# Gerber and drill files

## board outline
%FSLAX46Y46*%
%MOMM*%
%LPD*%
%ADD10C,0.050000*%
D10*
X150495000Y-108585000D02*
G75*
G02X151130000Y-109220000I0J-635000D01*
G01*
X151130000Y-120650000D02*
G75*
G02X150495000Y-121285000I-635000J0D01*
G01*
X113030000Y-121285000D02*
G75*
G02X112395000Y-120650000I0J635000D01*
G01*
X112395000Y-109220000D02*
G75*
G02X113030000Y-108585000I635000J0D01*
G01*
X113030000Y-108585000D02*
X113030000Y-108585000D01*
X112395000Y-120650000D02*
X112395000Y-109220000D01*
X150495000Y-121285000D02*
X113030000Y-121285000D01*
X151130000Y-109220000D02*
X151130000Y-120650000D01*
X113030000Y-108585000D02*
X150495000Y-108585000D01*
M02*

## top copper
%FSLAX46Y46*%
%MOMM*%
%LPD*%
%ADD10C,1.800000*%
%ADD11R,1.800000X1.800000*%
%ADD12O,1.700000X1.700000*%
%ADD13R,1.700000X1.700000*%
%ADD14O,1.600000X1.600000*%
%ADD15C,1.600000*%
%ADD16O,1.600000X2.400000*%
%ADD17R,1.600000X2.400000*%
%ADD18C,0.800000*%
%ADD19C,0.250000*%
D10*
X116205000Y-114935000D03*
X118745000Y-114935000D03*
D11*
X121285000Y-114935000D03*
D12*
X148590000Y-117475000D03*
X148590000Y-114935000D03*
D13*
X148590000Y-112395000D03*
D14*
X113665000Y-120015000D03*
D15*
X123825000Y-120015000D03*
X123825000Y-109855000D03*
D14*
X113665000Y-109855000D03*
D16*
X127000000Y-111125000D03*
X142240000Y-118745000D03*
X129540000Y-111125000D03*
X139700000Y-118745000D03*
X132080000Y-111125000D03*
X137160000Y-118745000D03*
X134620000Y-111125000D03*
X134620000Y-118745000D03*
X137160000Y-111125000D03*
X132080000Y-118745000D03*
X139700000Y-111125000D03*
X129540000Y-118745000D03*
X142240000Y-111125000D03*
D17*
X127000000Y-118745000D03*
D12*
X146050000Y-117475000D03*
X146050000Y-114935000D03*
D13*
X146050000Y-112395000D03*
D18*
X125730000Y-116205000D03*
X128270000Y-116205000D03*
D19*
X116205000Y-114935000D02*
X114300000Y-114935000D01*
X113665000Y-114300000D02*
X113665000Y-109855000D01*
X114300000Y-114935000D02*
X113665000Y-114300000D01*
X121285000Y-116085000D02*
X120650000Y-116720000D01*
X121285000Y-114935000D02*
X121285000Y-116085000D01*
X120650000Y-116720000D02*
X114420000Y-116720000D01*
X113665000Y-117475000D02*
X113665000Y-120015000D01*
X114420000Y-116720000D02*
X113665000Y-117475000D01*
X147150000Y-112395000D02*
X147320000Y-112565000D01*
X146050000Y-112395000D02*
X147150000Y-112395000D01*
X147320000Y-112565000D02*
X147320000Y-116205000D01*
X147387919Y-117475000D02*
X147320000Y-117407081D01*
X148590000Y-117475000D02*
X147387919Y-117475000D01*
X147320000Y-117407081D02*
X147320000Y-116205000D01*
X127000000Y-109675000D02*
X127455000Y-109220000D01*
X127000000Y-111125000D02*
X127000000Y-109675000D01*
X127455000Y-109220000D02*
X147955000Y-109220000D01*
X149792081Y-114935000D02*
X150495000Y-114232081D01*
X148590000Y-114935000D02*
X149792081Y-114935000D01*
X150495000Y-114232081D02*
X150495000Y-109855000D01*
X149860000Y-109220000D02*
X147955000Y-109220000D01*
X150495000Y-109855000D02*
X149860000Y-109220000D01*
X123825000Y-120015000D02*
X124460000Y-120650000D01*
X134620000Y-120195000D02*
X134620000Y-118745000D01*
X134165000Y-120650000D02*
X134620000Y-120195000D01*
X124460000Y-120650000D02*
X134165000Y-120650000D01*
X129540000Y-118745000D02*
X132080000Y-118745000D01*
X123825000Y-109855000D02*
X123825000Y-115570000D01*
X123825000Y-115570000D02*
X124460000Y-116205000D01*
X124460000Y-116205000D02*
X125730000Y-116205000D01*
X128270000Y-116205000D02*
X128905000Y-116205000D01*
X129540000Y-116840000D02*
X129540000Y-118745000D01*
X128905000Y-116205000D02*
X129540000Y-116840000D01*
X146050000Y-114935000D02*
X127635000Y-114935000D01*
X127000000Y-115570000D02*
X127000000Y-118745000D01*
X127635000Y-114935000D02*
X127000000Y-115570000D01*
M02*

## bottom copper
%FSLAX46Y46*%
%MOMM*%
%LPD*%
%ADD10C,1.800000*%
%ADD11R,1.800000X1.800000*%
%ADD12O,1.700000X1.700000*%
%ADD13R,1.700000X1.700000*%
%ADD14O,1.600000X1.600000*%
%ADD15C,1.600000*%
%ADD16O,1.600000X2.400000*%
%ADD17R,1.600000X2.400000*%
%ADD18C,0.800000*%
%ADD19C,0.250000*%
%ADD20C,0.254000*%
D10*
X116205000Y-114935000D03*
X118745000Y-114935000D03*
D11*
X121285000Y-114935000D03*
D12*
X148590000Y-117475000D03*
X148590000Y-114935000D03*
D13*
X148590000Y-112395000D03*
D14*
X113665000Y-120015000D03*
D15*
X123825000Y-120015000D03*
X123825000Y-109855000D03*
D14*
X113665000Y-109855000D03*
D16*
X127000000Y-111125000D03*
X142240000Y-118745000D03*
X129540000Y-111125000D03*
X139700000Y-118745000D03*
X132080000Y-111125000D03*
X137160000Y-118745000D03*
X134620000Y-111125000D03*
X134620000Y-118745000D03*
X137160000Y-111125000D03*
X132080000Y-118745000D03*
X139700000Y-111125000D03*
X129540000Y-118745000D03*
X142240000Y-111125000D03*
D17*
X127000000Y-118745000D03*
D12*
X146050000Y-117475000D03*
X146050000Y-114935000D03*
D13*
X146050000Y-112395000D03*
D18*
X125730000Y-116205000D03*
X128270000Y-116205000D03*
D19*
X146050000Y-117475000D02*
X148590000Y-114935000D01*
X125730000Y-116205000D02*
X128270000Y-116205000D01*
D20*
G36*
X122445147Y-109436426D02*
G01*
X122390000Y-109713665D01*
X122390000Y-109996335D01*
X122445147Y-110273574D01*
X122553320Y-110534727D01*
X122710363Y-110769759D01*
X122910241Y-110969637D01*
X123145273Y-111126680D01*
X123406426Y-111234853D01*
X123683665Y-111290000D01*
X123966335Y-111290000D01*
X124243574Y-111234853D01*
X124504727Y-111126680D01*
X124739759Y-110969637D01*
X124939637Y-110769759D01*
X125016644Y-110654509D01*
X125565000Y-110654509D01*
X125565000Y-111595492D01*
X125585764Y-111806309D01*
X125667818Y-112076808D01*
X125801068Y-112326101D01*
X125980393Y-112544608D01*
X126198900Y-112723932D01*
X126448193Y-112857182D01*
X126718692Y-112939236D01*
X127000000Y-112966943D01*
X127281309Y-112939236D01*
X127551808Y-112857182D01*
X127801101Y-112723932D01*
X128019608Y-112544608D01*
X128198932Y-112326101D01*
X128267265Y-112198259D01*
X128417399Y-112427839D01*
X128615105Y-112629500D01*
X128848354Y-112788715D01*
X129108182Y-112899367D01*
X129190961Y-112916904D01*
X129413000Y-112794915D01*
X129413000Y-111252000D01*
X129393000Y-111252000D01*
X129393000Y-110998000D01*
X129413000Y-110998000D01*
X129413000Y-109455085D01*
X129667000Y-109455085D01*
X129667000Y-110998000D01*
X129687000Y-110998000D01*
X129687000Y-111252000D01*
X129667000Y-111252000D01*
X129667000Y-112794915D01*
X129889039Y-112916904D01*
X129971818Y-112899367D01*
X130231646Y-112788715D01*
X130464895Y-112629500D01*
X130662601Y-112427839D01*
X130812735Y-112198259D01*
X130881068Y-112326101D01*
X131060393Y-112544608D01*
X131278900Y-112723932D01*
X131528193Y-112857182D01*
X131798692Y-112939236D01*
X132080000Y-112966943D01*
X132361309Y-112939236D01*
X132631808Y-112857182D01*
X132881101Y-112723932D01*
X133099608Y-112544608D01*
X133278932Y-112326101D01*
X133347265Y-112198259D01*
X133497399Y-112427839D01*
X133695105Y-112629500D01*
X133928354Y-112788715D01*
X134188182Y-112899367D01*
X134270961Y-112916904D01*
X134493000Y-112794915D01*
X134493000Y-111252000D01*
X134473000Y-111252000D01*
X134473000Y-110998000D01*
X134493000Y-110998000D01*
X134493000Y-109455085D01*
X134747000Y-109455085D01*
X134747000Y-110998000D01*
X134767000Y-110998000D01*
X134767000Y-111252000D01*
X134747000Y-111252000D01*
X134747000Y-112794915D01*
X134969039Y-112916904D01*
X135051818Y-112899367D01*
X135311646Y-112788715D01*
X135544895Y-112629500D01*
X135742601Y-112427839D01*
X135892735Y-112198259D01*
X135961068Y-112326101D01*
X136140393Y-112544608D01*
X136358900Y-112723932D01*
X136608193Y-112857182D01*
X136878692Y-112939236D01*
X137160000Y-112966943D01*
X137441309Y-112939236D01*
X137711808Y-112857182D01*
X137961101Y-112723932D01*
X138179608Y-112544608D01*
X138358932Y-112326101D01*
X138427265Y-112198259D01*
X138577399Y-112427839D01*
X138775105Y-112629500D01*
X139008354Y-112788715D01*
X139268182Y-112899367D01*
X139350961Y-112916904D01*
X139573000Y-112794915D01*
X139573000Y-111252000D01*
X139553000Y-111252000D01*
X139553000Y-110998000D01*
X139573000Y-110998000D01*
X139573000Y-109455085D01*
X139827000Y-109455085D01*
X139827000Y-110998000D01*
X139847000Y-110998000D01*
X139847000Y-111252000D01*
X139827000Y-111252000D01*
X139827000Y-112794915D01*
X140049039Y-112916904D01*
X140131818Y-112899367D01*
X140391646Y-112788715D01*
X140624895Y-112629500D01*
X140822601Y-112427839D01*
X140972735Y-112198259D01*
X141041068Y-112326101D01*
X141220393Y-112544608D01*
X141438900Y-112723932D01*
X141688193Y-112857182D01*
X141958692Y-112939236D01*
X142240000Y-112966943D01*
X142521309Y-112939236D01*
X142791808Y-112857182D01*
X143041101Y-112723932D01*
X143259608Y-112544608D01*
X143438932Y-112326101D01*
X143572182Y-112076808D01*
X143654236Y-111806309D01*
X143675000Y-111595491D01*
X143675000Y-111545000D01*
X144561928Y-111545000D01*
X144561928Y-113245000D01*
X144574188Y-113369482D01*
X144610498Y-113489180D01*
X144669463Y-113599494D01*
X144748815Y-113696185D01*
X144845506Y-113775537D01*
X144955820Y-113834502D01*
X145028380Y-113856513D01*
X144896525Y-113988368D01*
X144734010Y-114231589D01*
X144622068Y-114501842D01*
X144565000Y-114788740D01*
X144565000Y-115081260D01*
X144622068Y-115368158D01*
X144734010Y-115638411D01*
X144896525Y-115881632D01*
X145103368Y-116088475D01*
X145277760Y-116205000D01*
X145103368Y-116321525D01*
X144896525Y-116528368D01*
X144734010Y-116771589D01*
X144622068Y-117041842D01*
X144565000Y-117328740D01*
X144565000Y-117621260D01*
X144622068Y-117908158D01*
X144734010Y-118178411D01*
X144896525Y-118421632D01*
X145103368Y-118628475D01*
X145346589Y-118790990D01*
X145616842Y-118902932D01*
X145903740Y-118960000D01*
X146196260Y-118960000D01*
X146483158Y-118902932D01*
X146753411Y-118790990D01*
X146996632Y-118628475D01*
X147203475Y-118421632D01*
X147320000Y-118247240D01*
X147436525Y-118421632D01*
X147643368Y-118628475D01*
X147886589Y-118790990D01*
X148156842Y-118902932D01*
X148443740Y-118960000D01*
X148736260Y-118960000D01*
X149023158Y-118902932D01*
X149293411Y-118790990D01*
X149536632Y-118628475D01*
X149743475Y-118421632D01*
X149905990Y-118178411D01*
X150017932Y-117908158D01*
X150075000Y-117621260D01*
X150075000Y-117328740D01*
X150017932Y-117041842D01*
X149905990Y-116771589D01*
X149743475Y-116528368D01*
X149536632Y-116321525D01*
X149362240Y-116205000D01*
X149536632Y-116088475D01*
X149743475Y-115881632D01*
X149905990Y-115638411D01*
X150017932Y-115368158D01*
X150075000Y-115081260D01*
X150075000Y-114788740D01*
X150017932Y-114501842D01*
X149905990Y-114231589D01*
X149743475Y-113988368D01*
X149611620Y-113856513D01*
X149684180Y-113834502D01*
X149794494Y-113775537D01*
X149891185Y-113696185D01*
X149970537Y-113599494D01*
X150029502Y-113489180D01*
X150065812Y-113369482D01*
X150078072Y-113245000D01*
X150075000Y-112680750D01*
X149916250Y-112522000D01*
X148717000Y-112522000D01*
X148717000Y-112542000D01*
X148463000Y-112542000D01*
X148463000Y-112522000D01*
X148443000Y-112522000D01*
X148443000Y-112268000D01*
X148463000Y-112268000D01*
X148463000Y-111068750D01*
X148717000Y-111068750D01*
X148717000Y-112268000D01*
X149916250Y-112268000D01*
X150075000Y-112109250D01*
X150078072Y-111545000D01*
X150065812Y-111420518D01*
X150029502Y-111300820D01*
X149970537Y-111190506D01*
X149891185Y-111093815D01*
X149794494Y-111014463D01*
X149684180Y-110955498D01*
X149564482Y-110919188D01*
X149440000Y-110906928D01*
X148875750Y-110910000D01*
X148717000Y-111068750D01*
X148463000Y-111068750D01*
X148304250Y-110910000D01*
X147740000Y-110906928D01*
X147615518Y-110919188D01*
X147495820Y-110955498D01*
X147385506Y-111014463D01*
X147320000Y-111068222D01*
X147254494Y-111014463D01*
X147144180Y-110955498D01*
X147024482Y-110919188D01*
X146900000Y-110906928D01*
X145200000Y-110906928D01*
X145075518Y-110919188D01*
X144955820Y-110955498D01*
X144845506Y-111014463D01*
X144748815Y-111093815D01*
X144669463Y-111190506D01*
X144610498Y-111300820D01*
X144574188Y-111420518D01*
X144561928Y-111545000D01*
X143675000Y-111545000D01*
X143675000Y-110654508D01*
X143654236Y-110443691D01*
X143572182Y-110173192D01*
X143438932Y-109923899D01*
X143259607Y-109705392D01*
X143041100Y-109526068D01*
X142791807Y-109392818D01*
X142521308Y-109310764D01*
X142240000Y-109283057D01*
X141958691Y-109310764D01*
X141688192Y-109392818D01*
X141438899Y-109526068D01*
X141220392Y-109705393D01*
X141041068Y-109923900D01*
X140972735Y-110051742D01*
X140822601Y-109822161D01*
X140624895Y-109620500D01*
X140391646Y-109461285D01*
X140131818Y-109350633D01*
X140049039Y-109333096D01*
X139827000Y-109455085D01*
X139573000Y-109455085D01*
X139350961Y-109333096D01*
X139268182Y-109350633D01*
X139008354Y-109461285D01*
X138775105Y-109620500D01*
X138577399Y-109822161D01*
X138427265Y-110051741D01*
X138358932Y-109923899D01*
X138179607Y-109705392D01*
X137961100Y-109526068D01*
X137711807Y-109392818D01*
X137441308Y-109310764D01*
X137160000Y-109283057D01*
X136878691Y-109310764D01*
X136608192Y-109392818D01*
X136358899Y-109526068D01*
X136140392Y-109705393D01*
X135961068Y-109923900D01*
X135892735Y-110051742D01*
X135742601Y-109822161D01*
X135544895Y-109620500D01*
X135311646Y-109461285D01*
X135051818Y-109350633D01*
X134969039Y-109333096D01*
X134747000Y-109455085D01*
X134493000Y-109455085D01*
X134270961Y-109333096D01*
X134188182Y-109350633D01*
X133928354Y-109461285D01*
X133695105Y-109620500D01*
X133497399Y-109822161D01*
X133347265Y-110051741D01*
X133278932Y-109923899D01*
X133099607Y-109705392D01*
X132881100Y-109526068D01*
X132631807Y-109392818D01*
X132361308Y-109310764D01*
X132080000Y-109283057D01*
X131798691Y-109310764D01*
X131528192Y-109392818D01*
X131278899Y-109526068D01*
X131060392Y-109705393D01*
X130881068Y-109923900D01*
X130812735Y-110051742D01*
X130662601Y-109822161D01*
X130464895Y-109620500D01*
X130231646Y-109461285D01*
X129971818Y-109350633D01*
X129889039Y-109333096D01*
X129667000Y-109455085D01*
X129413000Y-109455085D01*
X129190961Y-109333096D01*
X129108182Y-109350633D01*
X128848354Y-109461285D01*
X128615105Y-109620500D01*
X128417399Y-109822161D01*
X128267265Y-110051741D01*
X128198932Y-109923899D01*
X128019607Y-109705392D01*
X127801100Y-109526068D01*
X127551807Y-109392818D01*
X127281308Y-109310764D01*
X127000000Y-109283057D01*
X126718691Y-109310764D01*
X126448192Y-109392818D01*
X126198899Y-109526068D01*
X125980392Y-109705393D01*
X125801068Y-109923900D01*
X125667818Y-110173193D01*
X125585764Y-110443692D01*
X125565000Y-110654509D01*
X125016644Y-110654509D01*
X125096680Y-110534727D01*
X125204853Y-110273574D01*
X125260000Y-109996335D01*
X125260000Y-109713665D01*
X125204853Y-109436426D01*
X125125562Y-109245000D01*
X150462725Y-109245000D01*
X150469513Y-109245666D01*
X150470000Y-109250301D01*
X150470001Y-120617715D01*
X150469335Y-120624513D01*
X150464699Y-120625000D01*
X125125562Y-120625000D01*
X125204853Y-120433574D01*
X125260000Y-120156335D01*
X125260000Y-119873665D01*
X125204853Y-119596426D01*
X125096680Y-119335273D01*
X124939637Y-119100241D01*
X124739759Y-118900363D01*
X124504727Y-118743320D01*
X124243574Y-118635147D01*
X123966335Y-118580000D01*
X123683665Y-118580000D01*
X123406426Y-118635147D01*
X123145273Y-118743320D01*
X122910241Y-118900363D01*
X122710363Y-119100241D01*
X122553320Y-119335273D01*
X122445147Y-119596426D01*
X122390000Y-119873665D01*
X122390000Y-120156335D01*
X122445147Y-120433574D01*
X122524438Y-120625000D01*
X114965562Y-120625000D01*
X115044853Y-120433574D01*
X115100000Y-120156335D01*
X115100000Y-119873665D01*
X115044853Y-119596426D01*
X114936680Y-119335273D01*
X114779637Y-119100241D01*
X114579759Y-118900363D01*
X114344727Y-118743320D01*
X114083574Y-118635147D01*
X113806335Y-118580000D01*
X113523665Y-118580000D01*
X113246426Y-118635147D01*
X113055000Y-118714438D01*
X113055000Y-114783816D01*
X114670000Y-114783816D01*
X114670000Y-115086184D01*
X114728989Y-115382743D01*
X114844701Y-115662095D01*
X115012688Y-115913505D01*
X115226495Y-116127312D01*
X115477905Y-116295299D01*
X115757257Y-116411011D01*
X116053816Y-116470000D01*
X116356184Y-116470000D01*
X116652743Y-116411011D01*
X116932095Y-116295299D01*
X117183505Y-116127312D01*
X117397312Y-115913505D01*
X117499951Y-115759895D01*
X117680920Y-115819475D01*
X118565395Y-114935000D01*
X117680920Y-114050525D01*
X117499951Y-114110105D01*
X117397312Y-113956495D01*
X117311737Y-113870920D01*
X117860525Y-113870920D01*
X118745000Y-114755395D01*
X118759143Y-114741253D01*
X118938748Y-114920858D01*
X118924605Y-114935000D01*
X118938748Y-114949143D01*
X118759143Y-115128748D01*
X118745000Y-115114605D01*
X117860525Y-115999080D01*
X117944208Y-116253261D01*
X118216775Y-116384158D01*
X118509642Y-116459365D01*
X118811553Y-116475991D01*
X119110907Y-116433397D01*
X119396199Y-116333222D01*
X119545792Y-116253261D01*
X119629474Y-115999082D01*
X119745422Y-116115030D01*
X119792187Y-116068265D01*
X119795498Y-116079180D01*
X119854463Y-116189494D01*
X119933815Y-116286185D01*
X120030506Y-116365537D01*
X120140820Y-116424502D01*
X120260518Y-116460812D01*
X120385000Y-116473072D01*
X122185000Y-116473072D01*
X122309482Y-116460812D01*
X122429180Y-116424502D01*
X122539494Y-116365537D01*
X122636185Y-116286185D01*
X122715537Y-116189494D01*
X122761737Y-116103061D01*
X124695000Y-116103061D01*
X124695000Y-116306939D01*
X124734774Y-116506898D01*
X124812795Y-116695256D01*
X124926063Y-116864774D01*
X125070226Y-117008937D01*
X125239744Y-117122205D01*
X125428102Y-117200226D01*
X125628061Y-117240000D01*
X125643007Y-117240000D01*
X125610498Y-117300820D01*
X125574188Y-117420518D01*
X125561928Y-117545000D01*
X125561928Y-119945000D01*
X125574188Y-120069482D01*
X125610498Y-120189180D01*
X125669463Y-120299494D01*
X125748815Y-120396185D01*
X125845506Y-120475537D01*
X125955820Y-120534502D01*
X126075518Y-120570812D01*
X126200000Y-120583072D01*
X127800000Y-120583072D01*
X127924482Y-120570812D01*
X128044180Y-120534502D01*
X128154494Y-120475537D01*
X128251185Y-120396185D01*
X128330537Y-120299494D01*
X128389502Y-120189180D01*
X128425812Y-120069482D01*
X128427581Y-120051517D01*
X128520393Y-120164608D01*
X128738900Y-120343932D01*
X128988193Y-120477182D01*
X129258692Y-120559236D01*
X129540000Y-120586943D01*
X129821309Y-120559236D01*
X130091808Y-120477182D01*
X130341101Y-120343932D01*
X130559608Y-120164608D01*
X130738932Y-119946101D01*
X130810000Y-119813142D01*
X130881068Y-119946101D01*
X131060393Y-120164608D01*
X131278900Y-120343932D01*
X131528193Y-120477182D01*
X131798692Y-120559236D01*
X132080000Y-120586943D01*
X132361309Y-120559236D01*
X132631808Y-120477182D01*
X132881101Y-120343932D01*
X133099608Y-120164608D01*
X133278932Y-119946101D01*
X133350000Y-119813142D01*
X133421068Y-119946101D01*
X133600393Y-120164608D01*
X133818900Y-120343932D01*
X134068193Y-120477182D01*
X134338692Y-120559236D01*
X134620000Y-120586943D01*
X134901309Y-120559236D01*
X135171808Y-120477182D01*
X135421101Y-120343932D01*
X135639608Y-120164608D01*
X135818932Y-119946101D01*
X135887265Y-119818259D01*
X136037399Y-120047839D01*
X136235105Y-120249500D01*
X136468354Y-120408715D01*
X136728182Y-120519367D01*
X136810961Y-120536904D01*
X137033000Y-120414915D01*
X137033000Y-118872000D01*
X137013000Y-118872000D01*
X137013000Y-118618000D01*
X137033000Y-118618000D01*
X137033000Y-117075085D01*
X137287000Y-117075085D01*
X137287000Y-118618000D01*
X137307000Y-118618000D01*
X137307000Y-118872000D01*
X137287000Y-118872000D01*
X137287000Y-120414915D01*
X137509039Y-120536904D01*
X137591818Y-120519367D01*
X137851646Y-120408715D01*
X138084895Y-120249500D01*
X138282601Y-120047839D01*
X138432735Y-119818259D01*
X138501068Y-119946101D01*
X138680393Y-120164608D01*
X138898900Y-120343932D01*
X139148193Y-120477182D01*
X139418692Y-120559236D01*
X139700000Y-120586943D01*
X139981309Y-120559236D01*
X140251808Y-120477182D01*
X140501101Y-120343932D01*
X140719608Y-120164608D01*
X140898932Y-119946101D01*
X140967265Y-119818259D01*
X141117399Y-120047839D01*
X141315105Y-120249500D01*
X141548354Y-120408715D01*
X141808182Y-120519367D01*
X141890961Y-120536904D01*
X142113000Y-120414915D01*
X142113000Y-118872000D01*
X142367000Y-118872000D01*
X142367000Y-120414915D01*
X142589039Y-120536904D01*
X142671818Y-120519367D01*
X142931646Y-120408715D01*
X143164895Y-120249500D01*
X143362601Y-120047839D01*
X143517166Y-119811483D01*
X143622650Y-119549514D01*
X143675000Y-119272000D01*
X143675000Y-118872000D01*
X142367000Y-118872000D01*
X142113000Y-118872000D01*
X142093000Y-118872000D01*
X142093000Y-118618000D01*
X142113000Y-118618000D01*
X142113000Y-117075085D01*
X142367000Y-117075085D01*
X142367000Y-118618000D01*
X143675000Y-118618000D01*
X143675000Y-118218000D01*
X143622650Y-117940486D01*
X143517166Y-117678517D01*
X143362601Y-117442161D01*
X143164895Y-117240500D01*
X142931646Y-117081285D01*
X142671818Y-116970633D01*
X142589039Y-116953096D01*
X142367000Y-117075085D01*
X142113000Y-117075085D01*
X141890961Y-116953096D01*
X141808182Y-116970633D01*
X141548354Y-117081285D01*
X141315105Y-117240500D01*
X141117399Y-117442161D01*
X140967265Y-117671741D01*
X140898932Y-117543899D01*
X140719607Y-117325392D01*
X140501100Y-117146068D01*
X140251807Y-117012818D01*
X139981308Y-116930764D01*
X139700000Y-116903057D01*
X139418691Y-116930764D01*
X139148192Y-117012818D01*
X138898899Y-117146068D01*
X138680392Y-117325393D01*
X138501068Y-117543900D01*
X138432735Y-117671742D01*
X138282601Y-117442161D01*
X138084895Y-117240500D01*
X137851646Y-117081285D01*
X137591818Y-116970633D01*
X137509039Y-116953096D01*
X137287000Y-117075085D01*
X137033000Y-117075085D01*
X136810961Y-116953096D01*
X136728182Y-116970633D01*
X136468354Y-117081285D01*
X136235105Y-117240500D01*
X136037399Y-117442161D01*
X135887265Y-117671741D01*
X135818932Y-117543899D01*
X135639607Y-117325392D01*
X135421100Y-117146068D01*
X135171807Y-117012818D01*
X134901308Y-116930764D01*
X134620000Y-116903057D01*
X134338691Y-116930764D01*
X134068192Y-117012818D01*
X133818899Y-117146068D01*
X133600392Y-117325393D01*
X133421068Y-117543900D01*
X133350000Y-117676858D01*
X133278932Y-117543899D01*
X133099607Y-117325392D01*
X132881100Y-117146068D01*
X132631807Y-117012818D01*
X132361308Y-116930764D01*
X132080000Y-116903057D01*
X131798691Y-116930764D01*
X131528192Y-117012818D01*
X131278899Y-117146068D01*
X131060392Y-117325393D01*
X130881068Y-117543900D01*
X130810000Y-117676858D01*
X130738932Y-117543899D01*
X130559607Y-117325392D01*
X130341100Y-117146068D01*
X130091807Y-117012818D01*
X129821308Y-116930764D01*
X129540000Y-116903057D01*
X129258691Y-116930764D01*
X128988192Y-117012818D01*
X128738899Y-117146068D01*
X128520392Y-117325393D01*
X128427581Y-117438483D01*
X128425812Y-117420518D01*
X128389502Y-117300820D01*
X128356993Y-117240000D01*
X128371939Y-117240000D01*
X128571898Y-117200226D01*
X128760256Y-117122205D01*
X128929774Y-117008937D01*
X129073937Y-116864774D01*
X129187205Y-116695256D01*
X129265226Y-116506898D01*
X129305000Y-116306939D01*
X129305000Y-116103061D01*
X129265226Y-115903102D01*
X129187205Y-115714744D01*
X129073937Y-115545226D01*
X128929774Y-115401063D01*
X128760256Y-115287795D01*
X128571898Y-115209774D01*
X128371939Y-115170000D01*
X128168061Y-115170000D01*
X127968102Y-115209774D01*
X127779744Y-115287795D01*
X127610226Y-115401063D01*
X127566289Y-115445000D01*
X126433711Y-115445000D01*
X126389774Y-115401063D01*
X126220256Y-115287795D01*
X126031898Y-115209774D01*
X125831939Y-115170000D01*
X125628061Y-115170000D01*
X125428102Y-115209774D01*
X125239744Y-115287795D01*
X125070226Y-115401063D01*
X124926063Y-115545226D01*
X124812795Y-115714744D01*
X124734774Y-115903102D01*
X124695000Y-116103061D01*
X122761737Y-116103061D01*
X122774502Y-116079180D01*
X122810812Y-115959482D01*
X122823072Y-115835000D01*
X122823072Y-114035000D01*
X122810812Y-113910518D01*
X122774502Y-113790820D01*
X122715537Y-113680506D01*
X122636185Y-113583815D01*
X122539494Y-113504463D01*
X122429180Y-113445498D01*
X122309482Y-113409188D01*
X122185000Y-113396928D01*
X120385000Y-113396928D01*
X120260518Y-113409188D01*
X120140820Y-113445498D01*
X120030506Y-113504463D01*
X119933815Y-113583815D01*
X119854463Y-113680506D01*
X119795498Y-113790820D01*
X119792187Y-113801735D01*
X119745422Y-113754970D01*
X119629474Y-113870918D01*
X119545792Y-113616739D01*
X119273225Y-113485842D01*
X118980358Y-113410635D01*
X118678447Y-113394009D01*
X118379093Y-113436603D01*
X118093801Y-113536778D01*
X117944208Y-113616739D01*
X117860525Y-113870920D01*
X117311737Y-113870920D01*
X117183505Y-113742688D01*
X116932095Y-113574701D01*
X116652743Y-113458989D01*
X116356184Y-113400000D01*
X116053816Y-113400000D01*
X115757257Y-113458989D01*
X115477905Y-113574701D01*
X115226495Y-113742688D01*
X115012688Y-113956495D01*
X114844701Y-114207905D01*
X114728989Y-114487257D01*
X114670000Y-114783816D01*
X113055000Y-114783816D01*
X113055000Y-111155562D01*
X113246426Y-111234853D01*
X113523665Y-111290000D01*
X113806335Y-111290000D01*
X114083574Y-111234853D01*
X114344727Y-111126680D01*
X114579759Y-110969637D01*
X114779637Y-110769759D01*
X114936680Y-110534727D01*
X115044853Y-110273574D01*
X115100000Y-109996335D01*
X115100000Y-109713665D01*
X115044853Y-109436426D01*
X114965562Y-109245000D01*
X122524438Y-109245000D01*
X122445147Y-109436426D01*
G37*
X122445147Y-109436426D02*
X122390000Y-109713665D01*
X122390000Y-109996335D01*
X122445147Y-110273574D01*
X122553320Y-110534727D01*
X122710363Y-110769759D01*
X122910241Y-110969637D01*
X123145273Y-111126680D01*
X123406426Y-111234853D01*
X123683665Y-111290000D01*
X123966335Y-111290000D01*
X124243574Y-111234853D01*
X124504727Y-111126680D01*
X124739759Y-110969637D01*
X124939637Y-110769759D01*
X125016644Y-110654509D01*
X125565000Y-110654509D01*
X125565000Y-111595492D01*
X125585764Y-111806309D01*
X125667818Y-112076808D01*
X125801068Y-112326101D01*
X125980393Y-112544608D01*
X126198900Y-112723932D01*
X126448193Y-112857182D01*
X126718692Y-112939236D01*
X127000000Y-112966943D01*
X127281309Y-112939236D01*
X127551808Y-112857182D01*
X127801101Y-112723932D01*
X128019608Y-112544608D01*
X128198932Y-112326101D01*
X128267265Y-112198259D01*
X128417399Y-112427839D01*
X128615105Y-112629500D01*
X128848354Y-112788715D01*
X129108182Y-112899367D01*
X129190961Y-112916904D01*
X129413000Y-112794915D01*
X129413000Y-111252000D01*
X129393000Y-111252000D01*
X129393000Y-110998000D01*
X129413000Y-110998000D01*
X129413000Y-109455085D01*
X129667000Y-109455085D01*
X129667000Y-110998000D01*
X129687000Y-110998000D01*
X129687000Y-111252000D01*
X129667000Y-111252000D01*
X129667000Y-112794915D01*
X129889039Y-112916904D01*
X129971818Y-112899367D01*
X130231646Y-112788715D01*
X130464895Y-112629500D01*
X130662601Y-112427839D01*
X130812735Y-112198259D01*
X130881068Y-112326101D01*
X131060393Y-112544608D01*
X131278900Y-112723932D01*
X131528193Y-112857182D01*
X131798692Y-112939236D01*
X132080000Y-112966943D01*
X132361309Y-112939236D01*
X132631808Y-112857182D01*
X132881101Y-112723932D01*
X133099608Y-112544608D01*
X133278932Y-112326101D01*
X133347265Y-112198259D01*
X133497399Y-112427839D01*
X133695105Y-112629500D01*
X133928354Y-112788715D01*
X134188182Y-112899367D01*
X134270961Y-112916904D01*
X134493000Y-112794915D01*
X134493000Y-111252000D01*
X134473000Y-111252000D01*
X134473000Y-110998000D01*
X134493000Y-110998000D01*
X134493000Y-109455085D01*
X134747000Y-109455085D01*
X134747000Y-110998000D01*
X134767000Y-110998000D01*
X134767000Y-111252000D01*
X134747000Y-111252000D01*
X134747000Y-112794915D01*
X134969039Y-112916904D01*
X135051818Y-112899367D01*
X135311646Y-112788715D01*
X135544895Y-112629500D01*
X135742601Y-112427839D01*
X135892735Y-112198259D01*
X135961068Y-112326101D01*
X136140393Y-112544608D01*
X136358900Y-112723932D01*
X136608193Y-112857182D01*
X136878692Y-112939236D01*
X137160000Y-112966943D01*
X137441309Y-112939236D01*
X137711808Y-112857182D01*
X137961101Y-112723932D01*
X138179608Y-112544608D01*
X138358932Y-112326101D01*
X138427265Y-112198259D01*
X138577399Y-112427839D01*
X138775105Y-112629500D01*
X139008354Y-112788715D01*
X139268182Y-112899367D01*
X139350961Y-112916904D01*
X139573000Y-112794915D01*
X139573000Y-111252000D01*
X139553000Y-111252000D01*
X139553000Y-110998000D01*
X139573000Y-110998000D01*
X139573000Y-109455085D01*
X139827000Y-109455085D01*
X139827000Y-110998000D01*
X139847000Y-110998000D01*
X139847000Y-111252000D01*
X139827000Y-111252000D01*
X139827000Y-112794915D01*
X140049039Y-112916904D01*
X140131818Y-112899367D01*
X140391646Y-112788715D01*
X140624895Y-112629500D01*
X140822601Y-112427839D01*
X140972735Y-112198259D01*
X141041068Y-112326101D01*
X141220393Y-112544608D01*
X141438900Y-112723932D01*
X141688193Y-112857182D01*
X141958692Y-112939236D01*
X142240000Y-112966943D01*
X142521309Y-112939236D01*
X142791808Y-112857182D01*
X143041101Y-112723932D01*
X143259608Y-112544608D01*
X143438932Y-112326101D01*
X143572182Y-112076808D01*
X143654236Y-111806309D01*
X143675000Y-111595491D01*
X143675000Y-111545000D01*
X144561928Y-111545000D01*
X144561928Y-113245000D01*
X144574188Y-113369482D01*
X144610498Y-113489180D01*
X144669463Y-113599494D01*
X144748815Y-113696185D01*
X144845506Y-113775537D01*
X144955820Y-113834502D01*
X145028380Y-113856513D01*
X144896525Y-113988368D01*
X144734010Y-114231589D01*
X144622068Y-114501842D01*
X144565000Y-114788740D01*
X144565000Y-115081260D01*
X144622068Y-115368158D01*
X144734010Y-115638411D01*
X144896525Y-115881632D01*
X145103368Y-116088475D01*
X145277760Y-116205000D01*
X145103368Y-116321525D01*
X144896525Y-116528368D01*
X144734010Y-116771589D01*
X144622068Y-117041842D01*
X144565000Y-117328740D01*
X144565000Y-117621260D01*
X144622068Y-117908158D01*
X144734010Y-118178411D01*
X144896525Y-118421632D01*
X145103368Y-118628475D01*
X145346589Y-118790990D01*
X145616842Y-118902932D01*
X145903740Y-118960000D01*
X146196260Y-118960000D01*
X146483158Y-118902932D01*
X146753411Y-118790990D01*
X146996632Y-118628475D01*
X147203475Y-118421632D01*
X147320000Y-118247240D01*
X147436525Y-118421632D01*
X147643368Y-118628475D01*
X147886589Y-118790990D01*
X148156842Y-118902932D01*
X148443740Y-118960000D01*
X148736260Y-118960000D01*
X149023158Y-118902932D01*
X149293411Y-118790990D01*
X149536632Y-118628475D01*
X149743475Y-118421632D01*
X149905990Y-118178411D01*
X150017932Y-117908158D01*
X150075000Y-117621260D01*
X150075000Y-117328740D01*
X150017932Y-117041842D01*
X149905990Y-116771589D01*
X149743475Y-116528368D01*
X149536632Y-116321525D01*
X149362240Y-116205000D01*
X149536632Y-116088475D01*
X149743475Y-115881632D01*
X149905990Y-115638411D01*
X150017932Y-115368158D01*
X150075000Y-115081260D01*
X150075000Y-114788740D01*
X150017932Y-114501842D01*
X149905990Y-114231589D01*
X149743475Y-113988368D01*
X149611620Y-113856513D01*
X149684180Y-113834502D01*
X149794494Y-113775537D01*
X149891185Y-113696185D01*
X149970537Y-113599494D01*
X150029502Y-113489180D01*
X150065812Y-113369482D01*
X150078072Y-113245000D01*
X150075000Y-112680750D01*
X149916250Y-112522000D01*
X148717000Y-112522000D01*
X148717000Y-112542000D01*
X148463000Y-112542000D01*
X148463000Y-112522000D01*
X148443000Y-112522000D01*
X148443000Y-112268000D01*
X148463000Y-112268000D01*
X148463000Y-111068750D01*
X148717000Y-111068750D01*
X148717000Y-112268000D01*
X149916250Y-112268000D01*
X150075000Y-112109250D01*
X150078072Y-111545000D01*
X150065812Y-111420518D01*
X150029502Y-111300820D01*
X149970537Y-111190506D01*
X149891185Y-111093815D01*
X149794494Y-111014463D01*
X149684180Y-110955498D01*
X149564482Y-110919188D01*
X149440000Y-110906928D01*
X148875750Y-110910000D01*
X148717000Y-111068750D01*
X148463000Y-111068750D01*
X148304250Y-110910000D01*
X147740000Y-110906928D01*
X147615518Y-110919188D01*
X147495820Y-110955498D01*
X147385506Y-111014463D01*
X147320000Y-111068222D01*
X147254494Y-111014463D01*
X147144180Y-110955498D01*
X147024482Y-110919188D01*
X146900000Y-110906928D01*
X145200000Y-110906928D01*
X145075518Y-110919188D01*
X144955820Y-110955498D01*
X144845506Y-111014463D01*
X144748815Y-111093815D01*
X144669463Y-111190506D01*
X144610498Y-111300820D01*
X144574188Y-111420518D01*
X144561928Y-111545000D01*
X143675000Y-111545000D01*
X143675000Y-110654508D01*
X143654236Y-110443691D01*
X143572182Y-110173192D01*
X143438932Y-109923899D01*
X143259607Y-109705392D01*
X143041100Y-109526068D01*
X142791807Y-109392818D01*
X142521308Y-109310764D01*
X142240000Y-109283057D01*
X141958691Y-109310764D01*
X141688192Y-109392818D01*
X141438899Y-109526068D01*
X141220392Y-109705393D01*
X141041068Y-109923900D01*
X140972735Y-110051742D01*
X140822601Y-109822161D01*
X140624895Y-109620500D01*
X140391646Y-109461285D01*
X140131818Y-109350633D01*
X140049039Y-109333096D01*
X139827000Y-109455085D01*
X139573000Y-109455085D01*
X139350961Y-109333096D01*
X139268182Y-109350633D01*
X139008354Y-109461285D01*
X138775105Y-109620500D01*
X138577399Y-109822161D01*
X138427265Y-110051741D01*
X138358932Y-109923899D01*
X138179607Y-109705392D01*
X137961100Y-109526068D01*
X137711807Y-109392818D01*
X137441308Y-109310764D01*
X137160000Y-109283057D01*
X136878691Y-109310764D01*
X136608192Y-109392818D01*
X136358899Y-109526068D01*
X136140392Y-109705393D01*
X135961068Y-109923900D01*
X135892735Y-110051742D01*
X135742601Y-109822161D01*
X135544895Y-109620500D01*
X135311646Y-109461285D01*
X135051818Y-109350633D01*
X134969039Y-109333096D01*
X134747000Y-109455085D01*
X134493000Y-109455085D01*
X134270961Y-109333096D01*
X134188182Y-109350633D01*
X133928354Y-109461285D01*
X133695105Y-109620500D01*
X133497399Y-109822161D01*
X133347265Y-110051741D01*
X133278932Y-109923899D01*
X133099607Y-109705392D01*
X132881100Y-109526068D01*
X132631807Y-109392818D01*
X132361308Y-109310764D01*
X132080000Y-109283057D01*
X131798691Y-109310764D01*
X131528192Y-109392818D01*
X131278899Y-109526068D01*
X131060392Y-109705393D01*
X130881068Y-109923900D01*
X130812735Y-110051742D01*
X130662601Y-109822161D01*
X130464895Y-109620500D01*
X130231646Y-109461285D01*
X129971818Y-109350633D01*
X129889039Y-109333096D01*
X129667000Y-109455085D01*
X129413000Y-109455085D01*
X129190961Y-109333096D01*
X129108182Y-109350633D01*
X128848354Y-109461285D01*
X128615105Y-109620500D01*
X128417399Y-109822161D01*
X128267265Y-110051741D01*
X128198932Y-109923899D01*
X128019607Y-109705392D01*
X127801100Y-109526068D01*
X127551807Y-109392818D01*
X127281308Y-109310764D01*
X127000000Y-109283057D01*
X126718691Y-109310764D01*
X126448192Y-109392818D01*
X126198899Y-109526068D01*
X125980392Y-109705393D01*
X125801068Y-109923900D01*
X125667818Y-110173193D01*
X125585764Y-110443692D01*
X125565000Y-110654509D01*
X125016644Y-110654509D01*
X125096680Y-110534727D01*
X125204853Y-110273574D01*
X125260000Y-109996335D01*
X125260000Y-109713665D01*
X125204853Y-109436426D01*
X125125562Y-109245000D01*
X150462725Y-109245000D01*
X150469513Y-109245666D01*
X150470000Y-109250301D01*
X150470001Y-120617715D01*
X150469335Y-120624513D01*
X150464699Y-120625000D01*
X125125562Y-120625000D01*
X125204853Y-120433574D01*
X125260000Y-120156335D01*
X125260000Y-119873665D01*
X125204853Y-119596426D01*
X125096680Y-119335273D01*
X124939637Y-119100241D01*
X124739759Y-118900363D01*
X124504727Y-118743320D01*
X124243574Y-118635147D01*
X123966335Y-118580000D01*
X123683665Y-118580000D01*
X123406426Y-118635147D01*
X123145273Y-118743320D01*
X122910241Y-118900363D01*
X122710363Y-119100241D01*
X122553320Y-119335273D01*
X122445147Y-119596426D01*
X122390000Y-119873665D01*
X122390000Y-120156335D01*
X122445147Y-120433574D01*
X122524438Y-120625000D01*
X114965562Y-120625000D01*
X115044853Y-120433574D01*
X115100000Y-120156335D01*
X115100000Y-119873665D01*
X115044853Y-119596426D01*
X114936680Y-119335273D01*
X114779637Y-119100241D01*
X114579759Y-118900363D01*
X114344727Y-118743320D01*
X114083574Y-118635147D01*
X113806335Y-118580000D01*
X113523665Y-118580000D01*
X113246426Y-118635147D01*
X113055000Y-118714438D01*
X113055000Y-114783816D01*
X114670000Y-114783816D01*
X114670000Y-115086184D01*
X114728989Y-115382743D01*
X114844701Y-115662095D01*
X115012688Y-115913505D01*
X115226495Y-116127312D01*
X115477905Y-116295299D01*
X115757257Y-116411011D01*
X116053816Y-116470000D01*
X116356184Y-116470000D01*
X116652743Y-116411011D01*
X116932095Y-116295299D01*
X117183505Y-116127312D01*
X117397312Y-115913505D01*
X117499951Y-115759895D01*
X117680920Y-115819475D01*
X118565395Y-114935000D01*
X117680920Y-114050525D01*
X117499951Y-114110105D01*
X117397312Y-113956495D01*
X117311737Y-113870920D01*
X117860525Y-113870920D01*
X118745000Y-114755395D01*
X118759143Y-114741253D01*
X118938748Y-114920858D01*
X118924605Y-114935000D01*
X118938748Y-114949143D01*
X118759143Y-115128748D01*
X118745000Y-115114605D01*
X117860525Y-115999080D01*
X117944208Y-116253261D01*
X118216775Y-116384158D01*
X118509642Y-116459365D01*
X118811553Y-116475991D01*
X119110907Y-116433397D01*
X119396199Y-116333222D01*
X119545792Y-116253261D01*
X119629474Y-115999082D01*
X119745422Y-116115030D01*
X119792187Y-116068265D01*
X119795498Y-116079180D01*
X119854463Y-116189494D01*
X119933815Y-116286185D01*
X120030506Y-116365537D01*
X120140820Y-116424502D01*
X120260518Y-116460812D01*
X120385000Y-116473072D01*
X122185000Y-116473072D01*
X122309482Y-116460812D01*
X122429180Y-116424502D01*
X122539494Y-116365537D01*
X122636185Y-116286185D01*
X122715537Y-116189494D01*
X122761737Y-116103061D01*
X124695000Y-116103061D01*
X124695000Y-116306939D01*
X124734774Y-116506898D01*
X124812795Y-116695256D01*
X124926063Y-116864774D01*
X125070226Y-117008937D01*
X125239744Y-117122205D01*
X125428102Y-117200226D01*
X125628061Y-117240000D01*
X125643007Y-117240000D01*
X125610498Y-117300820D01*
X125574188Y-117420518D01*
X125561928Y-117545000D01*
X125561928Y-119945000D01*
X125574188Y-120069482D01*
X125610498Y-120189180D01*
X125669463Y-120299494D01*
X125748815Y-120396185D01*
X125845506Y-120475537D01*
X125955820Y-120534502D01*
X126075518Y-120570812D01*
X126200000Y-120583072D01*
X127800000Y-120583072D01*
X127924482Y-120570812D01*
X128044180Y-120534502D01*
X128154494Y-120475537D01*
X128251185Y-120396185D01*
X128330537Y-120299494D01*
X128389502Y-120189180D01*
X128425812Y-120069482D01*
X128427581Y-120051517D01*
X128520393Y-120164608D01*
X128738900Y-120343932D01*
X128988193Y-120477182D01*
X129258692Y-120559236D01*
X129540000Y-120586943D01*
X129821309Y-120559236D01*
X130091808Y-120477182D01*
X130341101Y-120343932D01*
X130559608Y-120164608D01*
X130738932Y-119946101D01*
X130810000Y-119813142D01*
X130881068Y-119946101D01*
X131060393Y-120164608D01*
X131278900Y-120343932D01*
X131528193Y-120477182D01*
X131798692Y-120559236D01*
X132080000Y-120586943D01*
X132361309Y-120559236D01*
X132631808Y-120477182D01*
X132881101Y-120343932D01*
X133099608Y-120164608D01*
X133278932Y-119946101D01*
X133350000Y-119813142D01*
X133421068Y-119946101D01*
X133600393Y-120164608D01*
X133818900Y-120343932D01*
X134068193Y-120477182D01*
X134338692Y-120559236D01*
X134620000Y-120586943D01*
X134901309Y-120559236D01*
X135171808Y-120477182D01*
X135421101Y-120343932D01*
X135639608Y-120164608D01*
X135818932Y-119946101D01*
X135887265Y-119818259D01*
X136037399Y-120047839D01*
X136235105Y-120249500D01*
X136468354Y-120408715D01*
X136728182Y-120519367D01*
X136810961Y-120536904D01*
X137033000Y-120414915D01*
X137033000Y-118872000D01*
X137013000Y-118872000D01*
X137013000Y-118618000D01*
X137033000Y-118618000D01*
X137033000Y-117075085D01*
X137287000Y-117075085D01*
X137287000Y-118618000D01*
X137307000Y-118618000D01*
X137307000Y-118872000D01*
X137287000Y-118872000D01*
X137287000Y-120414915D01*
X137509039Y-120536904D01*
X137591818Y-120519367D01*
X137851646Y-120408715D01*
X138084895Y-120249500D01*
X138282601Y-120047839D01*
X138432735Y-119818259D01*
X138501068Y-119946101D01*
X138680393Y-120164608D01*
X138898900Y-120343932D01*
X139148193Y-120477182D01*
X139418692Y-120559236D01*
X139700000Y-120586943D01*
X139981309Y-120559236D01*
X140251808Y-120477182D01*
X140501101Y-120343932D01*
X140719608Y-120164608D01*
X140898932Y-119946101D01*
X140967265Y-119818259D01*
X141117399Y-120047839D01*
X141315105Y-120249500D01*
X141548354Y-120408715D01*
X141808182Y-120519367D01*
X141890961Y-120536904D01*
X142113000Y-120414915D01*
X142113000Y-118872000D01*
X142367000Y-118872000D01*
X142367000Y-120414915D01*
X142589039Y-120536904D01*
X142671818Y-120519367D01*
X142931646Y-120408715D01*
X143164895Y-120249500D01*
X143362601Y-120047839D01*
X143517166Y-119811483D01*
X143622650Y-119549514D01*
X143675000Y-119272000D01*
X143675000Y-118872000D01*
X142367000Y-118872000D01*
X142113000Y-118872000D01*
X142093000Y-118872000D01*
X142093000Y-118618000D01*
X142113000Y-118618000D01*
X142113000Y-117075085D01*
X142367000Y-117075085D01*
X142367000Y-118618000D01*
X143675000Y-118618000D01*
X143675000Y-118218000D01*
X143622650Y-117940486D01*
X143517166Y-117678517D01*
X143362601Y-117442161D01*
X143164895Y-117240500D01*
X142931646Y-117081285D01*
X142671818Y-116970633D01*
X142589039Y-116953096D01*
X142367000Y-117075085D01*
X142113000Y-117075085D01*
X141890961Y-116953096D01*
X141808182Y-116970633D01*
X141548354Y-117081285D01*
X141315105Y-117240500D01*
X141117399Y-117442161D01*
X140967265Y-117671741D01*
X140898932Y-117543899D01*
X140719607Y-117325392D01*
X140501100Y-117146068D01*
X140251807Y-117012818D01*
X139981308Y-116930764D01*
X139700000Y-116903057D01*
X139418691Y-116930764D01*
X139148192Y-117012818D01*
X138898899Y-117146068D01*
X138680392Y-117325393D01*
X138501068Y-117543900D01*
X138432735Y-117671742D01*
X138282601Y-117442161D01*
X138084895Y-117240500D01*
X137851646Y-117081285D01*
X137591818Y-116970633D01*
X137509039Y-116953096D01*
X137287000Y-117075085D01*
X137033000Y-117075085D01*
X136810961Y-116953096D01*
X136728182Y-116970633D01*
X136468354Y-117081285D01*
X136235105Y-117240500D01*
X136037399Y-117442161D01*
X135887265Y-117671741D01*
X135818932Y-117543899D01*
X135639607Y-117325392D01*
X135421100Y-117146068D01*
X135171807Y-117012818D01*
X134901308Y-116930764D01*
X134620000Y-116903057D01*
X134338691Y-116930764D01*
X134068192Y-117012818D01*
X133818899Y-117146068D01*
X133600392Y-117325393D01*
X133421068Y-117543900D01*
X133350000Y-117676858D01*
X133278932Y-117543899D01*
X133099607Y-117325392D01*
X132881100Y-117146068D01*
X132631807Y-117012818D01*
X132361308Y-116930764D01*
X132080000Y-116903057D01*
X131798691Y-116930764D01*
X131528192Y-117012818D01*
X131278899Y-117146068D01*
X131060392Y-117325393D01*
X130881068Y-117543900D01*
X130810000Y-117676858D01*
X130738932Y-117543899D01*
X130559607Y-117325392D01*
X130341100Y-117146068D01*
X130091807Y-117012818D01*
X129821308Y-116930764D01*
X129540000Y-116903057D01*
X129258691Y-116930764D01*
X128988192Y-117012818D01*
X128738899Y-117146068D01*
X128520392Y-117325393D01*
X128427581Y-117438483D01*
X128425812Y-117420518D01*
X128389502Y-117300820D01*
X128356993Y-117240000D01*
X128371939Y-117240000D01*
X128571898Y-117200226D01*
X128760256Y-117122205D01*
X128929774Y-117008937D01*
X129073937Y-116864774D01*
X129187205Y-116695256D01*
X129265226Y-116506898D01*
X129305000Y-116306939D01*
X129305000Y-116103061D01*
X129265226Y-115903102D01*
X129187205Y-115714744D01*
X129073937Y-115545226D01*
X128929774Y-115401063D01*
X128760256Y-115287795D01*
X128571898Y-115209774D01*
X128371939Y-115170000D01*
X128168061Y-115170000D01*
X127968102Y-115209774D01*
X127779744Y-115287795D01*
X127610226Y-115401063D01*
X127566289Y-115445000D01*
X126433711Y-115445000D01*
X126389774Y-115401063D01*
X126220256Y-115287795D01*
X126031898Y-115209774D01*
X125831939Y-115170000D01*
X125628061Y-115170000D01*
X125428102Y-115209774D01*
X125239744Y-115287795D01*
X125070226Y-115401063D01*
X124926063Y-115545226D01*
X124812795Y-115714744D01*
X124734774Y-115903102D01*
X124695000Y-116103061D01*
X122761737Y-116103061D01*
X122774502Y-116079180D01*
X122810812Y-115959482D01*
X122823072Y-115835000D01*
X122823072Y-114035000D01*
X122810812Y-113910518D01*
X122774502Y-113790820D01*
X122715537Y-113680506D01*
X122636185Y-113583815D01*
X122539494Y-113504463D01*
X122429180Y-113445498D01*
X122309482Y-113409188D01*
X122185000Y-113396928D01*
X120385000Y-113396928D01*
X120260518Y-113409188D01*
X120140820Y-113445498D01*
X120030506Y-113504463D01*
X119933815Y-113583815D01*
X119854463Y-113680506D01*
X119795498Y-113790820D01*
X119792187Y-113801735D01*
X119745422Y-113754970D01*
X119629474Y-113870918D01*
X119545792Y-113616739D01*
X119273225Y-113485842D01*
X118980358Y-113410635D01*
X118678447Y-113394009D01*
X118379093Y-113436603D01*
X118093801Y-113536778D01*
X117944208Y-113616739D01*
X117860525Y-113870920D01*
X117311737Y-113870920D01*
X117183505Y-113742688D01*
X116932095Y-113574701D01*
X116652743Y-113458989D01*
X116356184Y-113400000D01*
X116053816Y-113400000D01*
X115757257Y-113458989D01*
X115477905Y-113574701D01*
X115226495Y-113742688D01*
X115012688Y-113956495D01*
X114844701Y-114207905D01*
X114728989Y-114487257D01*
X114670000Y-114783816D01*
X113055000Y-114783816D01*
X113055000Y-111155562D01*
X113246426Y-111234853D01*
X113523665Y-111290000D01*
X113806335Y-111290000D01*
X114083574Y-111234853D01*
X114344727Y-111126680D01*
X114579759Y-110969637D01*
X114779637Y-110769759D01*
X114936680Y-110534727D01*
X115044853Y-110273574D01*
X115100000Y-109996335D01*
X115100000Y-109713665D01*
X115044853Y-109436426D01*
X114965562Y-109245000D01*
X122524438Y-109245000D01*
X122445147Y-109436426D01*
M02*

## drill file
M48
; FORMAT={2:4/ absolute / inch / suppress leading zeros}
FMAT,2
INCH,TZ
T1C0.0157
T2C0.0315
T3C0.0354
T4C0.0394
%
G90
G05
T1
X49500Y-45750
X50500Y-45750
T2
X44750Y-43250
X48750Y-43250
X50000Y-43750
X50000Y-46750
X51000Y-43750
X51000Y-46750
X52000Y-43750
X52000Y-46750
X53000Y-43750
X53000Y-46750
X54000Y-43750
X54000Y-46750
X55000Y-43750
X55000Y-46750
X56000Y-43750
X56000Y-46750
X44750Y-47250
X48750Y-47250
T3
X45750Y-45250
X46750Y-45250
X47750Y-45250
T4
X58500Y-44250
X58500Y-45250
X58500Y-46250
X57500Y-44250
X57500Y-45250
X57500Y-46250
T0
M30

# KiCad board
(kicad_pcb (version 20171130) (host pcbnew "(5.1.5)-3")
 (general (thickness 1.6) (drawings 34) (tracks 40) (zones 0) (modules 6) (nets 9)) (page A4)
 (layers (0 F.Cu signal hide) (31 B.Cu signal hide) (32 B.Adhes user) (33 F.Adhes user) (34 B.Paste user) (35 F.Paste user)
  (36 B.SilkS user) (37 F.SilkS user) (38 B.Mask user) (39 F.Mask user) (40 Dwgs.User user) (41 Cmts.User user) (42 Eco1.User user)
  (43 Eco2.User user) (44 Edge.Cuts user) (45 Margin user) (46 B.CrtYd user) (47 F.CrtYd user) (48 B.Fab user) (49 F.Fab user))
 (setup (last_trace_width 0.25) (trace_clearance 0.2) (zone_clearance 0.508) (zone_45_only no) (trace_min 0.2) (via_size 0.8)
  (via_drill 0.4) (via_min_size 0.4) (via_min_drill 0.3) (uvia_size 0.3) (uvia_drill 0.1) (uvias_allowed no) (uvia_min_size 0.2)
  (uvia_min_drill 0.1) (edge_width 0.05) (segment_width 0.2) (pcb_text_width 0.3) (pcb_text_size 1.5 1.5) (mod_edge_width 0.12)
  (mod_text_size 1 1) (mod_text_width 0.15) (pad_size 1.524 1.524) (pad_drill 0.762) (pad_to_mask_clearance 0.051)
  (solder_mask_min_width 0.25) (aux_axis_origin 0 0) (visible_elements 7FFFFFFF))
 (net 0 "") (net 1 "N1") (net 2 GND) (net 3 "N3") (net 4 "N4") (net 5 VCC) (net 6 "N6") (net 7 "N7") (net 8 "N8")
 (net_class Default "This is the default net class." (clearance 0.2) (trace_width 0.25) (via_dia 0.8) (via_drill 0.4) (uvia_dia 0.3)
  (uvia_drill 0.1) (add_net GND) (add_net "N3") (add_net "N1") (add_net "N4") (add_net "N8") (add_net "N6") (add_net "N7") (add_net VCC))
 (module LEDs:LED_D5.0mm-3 (layer F.Cu) (at 121.285 114.935 180)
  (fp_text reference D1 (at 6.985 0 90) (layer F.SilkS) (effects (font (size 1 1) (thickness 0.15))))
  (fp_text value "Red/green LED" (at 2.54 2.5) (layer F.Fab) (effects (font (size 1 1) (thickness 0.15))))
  (pad 3 thru_hole circle (at 5.08 0 180) (size 1.8 1.8) (drill 0.9) (layers *.Cu *.Mask) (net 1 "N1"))
  (pad 2 thru_hole circle (at 2.54 0 180) (size 1.8 1.8) (drill 0.9) (layers *.Cu *.Mask) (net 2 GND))
  (pad 1 thru_hole rect (at 0 0 180) (size 1.8 1.8) (drill 0.9) (layers *.Cu *.Mask) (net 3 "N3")))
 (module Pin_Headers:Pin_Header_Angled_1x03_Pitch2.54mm (layer F.Cu) (at 148.59 112.395)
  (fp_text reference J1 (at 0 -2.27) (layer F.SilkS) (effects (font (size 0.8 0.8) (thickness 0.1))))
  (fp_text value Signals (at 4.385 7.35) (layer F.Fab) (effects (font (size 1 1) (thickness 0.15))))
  (pad 3 thru_hole oval (at 0 5.08) (size 1.7 1.7) (drill 1) (layers *.Cu *.Mask) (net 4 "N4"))
  (pad 2 thru_hole oval (at 0 2.54) (size 1.7 1.7) (drill 1) (layers *.Cu *.Mask) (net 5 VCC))
  (pad 1 thru_hole rect (at 0 0) (size 1.7 1.7) (drill 1) (layers *.Cu *.Mask) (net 2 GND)))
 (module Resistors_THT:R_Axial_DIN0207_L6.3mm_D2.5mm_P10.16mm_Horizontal (layer F.Cu) (at 123.825 120.015 180)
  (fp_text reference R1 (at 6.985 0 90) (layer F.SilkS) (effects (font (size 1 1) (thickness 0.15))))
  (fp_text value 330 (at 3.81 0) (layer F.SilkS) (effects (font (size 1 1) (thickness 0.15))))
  (pad 2 thru_hole oval (at 10.16 0 180) (size 1.6 1.6) (drill 0.8) (layers *.Cu *.Mask) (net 3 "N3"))
  (pad 1 thru_hole circle (at 0 0 180) (size 1.6 1.6) (drill 0.8) (layers *.Cu *.Mask) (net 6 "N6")))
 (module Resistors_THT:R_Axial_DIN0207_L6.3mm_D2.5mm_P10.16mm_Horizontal (layer F.Cu) (at 123.825 109.855 180)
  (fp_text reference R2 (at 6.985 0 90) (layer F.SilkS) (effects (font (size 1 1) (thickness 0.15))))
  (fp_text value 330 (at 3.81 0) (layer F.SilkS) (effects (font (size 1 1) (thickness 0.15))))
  (pad 1 thru_hole circle (at 0 0 180) (size 1.6 1.6) (drill 0.8) (layers *.Cu *.Mask) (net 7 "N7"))
  (pad 2 thru_hole oval (at 10.16 0 180) (size 1.6 1.6) (drill 0.8) (layers *.Cu *.Mask) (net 1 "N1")))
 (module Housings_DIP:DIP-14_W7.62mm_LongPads (layer F.Cu) (at 127 118.745 90)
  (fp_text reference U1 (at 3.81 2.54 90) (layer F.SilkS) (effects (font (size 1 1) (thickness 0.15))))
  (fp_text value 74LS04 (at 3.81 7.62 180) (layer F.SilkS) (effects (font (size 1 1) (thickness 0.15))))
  (pad 14 thru_hole oval (at 7.62 0 90) (size 2.4 1.6) (drill 0.8) (layers *.Cu *.Mask) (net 5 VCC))
  (pad 7 thru_hole oval (at 0 15.24 90) (size 2.4 1.6) (drill 0.8) (layers *.Cu *.Mask) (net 2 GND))
  (pad 13 thru_hole oval (at 7.62 2.54 90) (size 2.4 1.6) (drill 0.8) (layers *.Cu *.Mask) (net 2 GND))
  (pad 6 thru_hole oval (at 0 12.7 90) (size 2.4 1.6) (drill 0.8) (layers *.Cu *.Mask))
  (pad 12 thru_hole oval (at 7.62 5.08 90) (size 2.4 1.6) (drill 0.8) (layers *.Cu *.Mask))
  (pad 5 thru_hole oval (at 0 10.16 90) (size 2.4 1.6) (drill 0.8) (layers *.Cu *.Mask) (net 2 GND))
  (pad 11 thru_hole oval (at 7.62 7.62 90) (size 2.4 1.6) (drill 0.8) (layers *.Cu *.Mask) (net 2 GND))
  (pad 4 thru_hole oval (at 0 7.62 90) (size 2.4 1.6) (drill 0.8) (layers *.Cu *.Mask) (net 6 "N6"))
  (pad 10 thru_hole oval (at 7.62 10.16 90) (size 2.4 1.6) (drill 0.8) (layers *.Cu *.Mask))
  (pad 3 thru_hole oval (at 0 5.08 90) (size 2.4 1.6) (drill 0.8) (layers *.Cu *.Mask) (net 7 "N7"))
  (pad 9 thru_hole oval (at 7.62 12.7 90) (size 2.4 1.6) (drill 0.8) (layers *.Cu *.Mask) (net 2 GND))
  (pad 2 thru_hole oval (at 0 2.54 90) (size 2.4 1.6) (drill 0.8) (layers *.Cu *.Mask) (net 7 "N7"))
  (pad 8 thru_hole oval (at 7.62 15.24 90) (size 2.4 1.6) (drill 0.8) (layers *.Cu *.Mask))
  (pad 1 thru_hole rect (at 0 0 90) (size 2.4 1.6) (drill 0.8) (layers *.Cu *.Mask) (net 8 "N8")))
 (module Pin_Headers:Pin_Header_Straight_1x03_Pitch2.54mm (layer F.Cu) (at 146.05 112.395)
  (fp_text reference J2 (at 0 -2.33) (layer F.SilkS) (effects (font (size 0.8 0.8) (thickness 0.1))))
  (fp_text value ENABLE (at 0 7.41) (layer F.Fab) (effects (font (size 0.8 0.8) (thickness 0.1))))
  (pad 3 thru_hole oval (at 0 5.08) (size 1.7 1.7) (drill 1) (layers *.Cu *.Mask) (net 5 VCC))
  (pad 2 thru_hole oval (at 0 2.54) (size 1.7 1.7) (drill 1) (layers *.Cu *.Mask) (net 8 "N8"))
  (pad 1 thru_hole rect (at 0 0) (size 1.7 1.7) (drill 1) (layers *.Cu *.Mask) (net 4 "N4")))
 (gr_arc (start 150.495 109.22) (end 151.13 109.22) (angle -90) (layer Edge.Cuts) (width 0.05))
 (gr_arc (start 150.495 120.65) (end 150.495 121.285) (angle -90) (layer Edge.Cuts) (width 0.05))
 (gr_arc (start 113.03 120.65) (end 112.395 120.65) (angle -90) (layer Edge.Cuts) (width 0.05))
 (gr_arc (start 113.03 109.22) (end 113.03 108.585) (angle -90) (layer Edge.Cuts) (width 0.05))
 (gr_line (start 113.03 108.585) (end 113.03 108.585) (layer Edge.Cuts) (width 0.05))
 (gr_line (start 112.395 120.65) (end 112.395 109.22) (layer Edge.Cuts) (width 0.05))
 (gr_line (start 150.495 121.285) (end 113.03 121.285) (layer Edge.Cuts) (width 0.05))
 (gr_line (start 151.13 109.22) (end 151.13 120.65) (layer Edge.Cuts) (width 0.05))
 (gr_line (start 113.03 108.585) (end 150.495 108.585) (layer Edge.Cuts) (width 0.05))
 (segment (start 116.205 114.935) (end 114.3 114.935) (width 0.25) (layer F.Cu) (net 1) (status 10))
 (segment (start 113.665 114.3) (end 113.665 109.855) (width 0.25) (layer F.Cu) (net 1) (status 20))
 (segment (start 114.3 114.935) (end 113.665 114.3) (width 0.25) (layer F.Cu) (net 1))
 (segment (start 121.285 116.085) (end 120.65 116.72) (width 0.25) (layer F.Cu) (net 3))
 (segment (start 121.285 114.935) (end 121.285 116.085) (width 0.25) (layer F.Cu) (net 3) (status 10))
 (segment (start 120.65 116.72) (end 114.42 116.72) (width 0.25) (layer F.Cu) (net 3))
 (segment (start 113.665 117.475) (end 113.665 120.015) (width 0.25) (layer F.Cu) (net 3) (status 20))
 (segment (start 114.42 116.72) (end 113.665 117.475) (width 0.25) (layer F.Cu) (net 3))
 (segment (start 147.15 112.395) (end 147.32 112.565) (width 0.25) (layer F.Cu) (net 4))
 (segment (start 146.05 112.395) (end 147.15 112.395) (width 0.25) (layer F.Cu) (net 4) (status 10))
 (segment (start 147.32 112.565) (end 147.32 116.205) (width 0.25) (layer F.Cu) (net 4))
 (segment (start 147.387919 117.475) (end 147.32 117.407081) (width 0.25) (layer F.Cu) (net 4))
 (segment (start 148.59 117.475) (end 147.387919 117.475) (width 0.25) (layer F.Cu) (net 4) (status 10))
 (segment (start 147.32 117.407081) (end 147.32 116.205) (width 0.25) (layer F.Cu) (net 4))
 (segment (start 127 109.675) (end 127.455 109.22) (width 0.25) (layer F.Cu) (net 5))
 (segment (start 127 111.125) (end 127 109.675) (width 0.25) (layer F.Cu) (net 5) (status 10))
 (segment (start 127.455 109.22) (end 147.955 109.22) (width 0.25) (layer F.Cu) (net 5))
 (segment (start 146.05 117.475) (end 148.59 114.935) (width 0.25) (layer B.Cu) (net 5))
 (segment (start 149.792081 114.935) (end 150.495 114.232081) (width 0.25) (layer F.Cu) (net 5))
 (segment (start 148.59 114.935) (end 149.792081 114.935) (width 0.25) (layer F.Cu) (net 5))
 (segment (start 150.495 114.232081) (end 150.495 109.855) (width 0.25) (layer F.Cu) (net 5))
 (segment (start 149.86 109.22) (end 147.955 109.22) (width 0.25) (layer F.Cu) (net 5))
 (segment (start 150.495 109.855) (end 149.86 109.22) (width 0.25) (layer F.Cu) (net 5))
 (segment (start 123.825 120.015) (end 124.46 120.65) (width 0.25) (layer F.Cu) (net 6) (status 10))
 (segment (start 134.62 120.195) (end 134.62 118.745) (width 0.25) (layer F.Cu) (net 6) (status 20))
 (segment (start 134.165 120.65) (end 134.62 120.195) (width 0.25) (layer F.Cu) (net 6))
 (segment (start 124.46 120.65) (end 134.165 120.65) (width 0.25) (layer F.Cu) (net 6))
 (segment (start 129.54 118.745) (end 132.08 118.745) (width 0.25) (layer F.Cu) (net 7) (status 30))
 (segment (start 123.825 109.855) (end 123.825 115.57) (width 0.25) (layer F.Cu) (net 7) (status 10))
 (via (at 125.73 116.205) (size 0.8) (drill 0.4) (layers F.Cu B.Cu) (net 7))
 (segment (start 123.825 115.57) (end 124.46 116.205) (width 0.25) (layer F.Cu) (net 7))
 (segment (start 124.46 116.205) (end 125.73 116.205) (width 0.25) (layer F.Cu) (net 7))
 (via (at 128.27 116.205) (size 0.8) (drill 0.4) (layers F.Cu B.Cu) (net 7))
 (segment (start 125.73 116.205) (end 128.27 116.205) (width 0.25) (layer B.Cu) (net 7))
 (segment (start 128.27 116.205) (end 128.905 116.205) (width 0.25) (layer F.Cu) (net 7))
 (segment (start 129.54 116.84) (end 129.54 118.745) (width 0.25) (layer F.Cu) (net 7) (status 20))
 (segment (start 128.905 116.205) (end 129.54 116.84) (width 0.25) (layer F.Cu) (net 7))
 (segment (start 146.05 114.935) (end 127.635 114.935) (width 0.25) (layer F.Cu) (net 8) (status 10))
 (segment (start 127 115.57) (end 127 118.745) (width 0.25) (layer F.Cu) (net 8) (status 20))
 (segment (start 127.635 114.935) (end 127 115.57) (width 0.25) (layer F.Cu) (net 8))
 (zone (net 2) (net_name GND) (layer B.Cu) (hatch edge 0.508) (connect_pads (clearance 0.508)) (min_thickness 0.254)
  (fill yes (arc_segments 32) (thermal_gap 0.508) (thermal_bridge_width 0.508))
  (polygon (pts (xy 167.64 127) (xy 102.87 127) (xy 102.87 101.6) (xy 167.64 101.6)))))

